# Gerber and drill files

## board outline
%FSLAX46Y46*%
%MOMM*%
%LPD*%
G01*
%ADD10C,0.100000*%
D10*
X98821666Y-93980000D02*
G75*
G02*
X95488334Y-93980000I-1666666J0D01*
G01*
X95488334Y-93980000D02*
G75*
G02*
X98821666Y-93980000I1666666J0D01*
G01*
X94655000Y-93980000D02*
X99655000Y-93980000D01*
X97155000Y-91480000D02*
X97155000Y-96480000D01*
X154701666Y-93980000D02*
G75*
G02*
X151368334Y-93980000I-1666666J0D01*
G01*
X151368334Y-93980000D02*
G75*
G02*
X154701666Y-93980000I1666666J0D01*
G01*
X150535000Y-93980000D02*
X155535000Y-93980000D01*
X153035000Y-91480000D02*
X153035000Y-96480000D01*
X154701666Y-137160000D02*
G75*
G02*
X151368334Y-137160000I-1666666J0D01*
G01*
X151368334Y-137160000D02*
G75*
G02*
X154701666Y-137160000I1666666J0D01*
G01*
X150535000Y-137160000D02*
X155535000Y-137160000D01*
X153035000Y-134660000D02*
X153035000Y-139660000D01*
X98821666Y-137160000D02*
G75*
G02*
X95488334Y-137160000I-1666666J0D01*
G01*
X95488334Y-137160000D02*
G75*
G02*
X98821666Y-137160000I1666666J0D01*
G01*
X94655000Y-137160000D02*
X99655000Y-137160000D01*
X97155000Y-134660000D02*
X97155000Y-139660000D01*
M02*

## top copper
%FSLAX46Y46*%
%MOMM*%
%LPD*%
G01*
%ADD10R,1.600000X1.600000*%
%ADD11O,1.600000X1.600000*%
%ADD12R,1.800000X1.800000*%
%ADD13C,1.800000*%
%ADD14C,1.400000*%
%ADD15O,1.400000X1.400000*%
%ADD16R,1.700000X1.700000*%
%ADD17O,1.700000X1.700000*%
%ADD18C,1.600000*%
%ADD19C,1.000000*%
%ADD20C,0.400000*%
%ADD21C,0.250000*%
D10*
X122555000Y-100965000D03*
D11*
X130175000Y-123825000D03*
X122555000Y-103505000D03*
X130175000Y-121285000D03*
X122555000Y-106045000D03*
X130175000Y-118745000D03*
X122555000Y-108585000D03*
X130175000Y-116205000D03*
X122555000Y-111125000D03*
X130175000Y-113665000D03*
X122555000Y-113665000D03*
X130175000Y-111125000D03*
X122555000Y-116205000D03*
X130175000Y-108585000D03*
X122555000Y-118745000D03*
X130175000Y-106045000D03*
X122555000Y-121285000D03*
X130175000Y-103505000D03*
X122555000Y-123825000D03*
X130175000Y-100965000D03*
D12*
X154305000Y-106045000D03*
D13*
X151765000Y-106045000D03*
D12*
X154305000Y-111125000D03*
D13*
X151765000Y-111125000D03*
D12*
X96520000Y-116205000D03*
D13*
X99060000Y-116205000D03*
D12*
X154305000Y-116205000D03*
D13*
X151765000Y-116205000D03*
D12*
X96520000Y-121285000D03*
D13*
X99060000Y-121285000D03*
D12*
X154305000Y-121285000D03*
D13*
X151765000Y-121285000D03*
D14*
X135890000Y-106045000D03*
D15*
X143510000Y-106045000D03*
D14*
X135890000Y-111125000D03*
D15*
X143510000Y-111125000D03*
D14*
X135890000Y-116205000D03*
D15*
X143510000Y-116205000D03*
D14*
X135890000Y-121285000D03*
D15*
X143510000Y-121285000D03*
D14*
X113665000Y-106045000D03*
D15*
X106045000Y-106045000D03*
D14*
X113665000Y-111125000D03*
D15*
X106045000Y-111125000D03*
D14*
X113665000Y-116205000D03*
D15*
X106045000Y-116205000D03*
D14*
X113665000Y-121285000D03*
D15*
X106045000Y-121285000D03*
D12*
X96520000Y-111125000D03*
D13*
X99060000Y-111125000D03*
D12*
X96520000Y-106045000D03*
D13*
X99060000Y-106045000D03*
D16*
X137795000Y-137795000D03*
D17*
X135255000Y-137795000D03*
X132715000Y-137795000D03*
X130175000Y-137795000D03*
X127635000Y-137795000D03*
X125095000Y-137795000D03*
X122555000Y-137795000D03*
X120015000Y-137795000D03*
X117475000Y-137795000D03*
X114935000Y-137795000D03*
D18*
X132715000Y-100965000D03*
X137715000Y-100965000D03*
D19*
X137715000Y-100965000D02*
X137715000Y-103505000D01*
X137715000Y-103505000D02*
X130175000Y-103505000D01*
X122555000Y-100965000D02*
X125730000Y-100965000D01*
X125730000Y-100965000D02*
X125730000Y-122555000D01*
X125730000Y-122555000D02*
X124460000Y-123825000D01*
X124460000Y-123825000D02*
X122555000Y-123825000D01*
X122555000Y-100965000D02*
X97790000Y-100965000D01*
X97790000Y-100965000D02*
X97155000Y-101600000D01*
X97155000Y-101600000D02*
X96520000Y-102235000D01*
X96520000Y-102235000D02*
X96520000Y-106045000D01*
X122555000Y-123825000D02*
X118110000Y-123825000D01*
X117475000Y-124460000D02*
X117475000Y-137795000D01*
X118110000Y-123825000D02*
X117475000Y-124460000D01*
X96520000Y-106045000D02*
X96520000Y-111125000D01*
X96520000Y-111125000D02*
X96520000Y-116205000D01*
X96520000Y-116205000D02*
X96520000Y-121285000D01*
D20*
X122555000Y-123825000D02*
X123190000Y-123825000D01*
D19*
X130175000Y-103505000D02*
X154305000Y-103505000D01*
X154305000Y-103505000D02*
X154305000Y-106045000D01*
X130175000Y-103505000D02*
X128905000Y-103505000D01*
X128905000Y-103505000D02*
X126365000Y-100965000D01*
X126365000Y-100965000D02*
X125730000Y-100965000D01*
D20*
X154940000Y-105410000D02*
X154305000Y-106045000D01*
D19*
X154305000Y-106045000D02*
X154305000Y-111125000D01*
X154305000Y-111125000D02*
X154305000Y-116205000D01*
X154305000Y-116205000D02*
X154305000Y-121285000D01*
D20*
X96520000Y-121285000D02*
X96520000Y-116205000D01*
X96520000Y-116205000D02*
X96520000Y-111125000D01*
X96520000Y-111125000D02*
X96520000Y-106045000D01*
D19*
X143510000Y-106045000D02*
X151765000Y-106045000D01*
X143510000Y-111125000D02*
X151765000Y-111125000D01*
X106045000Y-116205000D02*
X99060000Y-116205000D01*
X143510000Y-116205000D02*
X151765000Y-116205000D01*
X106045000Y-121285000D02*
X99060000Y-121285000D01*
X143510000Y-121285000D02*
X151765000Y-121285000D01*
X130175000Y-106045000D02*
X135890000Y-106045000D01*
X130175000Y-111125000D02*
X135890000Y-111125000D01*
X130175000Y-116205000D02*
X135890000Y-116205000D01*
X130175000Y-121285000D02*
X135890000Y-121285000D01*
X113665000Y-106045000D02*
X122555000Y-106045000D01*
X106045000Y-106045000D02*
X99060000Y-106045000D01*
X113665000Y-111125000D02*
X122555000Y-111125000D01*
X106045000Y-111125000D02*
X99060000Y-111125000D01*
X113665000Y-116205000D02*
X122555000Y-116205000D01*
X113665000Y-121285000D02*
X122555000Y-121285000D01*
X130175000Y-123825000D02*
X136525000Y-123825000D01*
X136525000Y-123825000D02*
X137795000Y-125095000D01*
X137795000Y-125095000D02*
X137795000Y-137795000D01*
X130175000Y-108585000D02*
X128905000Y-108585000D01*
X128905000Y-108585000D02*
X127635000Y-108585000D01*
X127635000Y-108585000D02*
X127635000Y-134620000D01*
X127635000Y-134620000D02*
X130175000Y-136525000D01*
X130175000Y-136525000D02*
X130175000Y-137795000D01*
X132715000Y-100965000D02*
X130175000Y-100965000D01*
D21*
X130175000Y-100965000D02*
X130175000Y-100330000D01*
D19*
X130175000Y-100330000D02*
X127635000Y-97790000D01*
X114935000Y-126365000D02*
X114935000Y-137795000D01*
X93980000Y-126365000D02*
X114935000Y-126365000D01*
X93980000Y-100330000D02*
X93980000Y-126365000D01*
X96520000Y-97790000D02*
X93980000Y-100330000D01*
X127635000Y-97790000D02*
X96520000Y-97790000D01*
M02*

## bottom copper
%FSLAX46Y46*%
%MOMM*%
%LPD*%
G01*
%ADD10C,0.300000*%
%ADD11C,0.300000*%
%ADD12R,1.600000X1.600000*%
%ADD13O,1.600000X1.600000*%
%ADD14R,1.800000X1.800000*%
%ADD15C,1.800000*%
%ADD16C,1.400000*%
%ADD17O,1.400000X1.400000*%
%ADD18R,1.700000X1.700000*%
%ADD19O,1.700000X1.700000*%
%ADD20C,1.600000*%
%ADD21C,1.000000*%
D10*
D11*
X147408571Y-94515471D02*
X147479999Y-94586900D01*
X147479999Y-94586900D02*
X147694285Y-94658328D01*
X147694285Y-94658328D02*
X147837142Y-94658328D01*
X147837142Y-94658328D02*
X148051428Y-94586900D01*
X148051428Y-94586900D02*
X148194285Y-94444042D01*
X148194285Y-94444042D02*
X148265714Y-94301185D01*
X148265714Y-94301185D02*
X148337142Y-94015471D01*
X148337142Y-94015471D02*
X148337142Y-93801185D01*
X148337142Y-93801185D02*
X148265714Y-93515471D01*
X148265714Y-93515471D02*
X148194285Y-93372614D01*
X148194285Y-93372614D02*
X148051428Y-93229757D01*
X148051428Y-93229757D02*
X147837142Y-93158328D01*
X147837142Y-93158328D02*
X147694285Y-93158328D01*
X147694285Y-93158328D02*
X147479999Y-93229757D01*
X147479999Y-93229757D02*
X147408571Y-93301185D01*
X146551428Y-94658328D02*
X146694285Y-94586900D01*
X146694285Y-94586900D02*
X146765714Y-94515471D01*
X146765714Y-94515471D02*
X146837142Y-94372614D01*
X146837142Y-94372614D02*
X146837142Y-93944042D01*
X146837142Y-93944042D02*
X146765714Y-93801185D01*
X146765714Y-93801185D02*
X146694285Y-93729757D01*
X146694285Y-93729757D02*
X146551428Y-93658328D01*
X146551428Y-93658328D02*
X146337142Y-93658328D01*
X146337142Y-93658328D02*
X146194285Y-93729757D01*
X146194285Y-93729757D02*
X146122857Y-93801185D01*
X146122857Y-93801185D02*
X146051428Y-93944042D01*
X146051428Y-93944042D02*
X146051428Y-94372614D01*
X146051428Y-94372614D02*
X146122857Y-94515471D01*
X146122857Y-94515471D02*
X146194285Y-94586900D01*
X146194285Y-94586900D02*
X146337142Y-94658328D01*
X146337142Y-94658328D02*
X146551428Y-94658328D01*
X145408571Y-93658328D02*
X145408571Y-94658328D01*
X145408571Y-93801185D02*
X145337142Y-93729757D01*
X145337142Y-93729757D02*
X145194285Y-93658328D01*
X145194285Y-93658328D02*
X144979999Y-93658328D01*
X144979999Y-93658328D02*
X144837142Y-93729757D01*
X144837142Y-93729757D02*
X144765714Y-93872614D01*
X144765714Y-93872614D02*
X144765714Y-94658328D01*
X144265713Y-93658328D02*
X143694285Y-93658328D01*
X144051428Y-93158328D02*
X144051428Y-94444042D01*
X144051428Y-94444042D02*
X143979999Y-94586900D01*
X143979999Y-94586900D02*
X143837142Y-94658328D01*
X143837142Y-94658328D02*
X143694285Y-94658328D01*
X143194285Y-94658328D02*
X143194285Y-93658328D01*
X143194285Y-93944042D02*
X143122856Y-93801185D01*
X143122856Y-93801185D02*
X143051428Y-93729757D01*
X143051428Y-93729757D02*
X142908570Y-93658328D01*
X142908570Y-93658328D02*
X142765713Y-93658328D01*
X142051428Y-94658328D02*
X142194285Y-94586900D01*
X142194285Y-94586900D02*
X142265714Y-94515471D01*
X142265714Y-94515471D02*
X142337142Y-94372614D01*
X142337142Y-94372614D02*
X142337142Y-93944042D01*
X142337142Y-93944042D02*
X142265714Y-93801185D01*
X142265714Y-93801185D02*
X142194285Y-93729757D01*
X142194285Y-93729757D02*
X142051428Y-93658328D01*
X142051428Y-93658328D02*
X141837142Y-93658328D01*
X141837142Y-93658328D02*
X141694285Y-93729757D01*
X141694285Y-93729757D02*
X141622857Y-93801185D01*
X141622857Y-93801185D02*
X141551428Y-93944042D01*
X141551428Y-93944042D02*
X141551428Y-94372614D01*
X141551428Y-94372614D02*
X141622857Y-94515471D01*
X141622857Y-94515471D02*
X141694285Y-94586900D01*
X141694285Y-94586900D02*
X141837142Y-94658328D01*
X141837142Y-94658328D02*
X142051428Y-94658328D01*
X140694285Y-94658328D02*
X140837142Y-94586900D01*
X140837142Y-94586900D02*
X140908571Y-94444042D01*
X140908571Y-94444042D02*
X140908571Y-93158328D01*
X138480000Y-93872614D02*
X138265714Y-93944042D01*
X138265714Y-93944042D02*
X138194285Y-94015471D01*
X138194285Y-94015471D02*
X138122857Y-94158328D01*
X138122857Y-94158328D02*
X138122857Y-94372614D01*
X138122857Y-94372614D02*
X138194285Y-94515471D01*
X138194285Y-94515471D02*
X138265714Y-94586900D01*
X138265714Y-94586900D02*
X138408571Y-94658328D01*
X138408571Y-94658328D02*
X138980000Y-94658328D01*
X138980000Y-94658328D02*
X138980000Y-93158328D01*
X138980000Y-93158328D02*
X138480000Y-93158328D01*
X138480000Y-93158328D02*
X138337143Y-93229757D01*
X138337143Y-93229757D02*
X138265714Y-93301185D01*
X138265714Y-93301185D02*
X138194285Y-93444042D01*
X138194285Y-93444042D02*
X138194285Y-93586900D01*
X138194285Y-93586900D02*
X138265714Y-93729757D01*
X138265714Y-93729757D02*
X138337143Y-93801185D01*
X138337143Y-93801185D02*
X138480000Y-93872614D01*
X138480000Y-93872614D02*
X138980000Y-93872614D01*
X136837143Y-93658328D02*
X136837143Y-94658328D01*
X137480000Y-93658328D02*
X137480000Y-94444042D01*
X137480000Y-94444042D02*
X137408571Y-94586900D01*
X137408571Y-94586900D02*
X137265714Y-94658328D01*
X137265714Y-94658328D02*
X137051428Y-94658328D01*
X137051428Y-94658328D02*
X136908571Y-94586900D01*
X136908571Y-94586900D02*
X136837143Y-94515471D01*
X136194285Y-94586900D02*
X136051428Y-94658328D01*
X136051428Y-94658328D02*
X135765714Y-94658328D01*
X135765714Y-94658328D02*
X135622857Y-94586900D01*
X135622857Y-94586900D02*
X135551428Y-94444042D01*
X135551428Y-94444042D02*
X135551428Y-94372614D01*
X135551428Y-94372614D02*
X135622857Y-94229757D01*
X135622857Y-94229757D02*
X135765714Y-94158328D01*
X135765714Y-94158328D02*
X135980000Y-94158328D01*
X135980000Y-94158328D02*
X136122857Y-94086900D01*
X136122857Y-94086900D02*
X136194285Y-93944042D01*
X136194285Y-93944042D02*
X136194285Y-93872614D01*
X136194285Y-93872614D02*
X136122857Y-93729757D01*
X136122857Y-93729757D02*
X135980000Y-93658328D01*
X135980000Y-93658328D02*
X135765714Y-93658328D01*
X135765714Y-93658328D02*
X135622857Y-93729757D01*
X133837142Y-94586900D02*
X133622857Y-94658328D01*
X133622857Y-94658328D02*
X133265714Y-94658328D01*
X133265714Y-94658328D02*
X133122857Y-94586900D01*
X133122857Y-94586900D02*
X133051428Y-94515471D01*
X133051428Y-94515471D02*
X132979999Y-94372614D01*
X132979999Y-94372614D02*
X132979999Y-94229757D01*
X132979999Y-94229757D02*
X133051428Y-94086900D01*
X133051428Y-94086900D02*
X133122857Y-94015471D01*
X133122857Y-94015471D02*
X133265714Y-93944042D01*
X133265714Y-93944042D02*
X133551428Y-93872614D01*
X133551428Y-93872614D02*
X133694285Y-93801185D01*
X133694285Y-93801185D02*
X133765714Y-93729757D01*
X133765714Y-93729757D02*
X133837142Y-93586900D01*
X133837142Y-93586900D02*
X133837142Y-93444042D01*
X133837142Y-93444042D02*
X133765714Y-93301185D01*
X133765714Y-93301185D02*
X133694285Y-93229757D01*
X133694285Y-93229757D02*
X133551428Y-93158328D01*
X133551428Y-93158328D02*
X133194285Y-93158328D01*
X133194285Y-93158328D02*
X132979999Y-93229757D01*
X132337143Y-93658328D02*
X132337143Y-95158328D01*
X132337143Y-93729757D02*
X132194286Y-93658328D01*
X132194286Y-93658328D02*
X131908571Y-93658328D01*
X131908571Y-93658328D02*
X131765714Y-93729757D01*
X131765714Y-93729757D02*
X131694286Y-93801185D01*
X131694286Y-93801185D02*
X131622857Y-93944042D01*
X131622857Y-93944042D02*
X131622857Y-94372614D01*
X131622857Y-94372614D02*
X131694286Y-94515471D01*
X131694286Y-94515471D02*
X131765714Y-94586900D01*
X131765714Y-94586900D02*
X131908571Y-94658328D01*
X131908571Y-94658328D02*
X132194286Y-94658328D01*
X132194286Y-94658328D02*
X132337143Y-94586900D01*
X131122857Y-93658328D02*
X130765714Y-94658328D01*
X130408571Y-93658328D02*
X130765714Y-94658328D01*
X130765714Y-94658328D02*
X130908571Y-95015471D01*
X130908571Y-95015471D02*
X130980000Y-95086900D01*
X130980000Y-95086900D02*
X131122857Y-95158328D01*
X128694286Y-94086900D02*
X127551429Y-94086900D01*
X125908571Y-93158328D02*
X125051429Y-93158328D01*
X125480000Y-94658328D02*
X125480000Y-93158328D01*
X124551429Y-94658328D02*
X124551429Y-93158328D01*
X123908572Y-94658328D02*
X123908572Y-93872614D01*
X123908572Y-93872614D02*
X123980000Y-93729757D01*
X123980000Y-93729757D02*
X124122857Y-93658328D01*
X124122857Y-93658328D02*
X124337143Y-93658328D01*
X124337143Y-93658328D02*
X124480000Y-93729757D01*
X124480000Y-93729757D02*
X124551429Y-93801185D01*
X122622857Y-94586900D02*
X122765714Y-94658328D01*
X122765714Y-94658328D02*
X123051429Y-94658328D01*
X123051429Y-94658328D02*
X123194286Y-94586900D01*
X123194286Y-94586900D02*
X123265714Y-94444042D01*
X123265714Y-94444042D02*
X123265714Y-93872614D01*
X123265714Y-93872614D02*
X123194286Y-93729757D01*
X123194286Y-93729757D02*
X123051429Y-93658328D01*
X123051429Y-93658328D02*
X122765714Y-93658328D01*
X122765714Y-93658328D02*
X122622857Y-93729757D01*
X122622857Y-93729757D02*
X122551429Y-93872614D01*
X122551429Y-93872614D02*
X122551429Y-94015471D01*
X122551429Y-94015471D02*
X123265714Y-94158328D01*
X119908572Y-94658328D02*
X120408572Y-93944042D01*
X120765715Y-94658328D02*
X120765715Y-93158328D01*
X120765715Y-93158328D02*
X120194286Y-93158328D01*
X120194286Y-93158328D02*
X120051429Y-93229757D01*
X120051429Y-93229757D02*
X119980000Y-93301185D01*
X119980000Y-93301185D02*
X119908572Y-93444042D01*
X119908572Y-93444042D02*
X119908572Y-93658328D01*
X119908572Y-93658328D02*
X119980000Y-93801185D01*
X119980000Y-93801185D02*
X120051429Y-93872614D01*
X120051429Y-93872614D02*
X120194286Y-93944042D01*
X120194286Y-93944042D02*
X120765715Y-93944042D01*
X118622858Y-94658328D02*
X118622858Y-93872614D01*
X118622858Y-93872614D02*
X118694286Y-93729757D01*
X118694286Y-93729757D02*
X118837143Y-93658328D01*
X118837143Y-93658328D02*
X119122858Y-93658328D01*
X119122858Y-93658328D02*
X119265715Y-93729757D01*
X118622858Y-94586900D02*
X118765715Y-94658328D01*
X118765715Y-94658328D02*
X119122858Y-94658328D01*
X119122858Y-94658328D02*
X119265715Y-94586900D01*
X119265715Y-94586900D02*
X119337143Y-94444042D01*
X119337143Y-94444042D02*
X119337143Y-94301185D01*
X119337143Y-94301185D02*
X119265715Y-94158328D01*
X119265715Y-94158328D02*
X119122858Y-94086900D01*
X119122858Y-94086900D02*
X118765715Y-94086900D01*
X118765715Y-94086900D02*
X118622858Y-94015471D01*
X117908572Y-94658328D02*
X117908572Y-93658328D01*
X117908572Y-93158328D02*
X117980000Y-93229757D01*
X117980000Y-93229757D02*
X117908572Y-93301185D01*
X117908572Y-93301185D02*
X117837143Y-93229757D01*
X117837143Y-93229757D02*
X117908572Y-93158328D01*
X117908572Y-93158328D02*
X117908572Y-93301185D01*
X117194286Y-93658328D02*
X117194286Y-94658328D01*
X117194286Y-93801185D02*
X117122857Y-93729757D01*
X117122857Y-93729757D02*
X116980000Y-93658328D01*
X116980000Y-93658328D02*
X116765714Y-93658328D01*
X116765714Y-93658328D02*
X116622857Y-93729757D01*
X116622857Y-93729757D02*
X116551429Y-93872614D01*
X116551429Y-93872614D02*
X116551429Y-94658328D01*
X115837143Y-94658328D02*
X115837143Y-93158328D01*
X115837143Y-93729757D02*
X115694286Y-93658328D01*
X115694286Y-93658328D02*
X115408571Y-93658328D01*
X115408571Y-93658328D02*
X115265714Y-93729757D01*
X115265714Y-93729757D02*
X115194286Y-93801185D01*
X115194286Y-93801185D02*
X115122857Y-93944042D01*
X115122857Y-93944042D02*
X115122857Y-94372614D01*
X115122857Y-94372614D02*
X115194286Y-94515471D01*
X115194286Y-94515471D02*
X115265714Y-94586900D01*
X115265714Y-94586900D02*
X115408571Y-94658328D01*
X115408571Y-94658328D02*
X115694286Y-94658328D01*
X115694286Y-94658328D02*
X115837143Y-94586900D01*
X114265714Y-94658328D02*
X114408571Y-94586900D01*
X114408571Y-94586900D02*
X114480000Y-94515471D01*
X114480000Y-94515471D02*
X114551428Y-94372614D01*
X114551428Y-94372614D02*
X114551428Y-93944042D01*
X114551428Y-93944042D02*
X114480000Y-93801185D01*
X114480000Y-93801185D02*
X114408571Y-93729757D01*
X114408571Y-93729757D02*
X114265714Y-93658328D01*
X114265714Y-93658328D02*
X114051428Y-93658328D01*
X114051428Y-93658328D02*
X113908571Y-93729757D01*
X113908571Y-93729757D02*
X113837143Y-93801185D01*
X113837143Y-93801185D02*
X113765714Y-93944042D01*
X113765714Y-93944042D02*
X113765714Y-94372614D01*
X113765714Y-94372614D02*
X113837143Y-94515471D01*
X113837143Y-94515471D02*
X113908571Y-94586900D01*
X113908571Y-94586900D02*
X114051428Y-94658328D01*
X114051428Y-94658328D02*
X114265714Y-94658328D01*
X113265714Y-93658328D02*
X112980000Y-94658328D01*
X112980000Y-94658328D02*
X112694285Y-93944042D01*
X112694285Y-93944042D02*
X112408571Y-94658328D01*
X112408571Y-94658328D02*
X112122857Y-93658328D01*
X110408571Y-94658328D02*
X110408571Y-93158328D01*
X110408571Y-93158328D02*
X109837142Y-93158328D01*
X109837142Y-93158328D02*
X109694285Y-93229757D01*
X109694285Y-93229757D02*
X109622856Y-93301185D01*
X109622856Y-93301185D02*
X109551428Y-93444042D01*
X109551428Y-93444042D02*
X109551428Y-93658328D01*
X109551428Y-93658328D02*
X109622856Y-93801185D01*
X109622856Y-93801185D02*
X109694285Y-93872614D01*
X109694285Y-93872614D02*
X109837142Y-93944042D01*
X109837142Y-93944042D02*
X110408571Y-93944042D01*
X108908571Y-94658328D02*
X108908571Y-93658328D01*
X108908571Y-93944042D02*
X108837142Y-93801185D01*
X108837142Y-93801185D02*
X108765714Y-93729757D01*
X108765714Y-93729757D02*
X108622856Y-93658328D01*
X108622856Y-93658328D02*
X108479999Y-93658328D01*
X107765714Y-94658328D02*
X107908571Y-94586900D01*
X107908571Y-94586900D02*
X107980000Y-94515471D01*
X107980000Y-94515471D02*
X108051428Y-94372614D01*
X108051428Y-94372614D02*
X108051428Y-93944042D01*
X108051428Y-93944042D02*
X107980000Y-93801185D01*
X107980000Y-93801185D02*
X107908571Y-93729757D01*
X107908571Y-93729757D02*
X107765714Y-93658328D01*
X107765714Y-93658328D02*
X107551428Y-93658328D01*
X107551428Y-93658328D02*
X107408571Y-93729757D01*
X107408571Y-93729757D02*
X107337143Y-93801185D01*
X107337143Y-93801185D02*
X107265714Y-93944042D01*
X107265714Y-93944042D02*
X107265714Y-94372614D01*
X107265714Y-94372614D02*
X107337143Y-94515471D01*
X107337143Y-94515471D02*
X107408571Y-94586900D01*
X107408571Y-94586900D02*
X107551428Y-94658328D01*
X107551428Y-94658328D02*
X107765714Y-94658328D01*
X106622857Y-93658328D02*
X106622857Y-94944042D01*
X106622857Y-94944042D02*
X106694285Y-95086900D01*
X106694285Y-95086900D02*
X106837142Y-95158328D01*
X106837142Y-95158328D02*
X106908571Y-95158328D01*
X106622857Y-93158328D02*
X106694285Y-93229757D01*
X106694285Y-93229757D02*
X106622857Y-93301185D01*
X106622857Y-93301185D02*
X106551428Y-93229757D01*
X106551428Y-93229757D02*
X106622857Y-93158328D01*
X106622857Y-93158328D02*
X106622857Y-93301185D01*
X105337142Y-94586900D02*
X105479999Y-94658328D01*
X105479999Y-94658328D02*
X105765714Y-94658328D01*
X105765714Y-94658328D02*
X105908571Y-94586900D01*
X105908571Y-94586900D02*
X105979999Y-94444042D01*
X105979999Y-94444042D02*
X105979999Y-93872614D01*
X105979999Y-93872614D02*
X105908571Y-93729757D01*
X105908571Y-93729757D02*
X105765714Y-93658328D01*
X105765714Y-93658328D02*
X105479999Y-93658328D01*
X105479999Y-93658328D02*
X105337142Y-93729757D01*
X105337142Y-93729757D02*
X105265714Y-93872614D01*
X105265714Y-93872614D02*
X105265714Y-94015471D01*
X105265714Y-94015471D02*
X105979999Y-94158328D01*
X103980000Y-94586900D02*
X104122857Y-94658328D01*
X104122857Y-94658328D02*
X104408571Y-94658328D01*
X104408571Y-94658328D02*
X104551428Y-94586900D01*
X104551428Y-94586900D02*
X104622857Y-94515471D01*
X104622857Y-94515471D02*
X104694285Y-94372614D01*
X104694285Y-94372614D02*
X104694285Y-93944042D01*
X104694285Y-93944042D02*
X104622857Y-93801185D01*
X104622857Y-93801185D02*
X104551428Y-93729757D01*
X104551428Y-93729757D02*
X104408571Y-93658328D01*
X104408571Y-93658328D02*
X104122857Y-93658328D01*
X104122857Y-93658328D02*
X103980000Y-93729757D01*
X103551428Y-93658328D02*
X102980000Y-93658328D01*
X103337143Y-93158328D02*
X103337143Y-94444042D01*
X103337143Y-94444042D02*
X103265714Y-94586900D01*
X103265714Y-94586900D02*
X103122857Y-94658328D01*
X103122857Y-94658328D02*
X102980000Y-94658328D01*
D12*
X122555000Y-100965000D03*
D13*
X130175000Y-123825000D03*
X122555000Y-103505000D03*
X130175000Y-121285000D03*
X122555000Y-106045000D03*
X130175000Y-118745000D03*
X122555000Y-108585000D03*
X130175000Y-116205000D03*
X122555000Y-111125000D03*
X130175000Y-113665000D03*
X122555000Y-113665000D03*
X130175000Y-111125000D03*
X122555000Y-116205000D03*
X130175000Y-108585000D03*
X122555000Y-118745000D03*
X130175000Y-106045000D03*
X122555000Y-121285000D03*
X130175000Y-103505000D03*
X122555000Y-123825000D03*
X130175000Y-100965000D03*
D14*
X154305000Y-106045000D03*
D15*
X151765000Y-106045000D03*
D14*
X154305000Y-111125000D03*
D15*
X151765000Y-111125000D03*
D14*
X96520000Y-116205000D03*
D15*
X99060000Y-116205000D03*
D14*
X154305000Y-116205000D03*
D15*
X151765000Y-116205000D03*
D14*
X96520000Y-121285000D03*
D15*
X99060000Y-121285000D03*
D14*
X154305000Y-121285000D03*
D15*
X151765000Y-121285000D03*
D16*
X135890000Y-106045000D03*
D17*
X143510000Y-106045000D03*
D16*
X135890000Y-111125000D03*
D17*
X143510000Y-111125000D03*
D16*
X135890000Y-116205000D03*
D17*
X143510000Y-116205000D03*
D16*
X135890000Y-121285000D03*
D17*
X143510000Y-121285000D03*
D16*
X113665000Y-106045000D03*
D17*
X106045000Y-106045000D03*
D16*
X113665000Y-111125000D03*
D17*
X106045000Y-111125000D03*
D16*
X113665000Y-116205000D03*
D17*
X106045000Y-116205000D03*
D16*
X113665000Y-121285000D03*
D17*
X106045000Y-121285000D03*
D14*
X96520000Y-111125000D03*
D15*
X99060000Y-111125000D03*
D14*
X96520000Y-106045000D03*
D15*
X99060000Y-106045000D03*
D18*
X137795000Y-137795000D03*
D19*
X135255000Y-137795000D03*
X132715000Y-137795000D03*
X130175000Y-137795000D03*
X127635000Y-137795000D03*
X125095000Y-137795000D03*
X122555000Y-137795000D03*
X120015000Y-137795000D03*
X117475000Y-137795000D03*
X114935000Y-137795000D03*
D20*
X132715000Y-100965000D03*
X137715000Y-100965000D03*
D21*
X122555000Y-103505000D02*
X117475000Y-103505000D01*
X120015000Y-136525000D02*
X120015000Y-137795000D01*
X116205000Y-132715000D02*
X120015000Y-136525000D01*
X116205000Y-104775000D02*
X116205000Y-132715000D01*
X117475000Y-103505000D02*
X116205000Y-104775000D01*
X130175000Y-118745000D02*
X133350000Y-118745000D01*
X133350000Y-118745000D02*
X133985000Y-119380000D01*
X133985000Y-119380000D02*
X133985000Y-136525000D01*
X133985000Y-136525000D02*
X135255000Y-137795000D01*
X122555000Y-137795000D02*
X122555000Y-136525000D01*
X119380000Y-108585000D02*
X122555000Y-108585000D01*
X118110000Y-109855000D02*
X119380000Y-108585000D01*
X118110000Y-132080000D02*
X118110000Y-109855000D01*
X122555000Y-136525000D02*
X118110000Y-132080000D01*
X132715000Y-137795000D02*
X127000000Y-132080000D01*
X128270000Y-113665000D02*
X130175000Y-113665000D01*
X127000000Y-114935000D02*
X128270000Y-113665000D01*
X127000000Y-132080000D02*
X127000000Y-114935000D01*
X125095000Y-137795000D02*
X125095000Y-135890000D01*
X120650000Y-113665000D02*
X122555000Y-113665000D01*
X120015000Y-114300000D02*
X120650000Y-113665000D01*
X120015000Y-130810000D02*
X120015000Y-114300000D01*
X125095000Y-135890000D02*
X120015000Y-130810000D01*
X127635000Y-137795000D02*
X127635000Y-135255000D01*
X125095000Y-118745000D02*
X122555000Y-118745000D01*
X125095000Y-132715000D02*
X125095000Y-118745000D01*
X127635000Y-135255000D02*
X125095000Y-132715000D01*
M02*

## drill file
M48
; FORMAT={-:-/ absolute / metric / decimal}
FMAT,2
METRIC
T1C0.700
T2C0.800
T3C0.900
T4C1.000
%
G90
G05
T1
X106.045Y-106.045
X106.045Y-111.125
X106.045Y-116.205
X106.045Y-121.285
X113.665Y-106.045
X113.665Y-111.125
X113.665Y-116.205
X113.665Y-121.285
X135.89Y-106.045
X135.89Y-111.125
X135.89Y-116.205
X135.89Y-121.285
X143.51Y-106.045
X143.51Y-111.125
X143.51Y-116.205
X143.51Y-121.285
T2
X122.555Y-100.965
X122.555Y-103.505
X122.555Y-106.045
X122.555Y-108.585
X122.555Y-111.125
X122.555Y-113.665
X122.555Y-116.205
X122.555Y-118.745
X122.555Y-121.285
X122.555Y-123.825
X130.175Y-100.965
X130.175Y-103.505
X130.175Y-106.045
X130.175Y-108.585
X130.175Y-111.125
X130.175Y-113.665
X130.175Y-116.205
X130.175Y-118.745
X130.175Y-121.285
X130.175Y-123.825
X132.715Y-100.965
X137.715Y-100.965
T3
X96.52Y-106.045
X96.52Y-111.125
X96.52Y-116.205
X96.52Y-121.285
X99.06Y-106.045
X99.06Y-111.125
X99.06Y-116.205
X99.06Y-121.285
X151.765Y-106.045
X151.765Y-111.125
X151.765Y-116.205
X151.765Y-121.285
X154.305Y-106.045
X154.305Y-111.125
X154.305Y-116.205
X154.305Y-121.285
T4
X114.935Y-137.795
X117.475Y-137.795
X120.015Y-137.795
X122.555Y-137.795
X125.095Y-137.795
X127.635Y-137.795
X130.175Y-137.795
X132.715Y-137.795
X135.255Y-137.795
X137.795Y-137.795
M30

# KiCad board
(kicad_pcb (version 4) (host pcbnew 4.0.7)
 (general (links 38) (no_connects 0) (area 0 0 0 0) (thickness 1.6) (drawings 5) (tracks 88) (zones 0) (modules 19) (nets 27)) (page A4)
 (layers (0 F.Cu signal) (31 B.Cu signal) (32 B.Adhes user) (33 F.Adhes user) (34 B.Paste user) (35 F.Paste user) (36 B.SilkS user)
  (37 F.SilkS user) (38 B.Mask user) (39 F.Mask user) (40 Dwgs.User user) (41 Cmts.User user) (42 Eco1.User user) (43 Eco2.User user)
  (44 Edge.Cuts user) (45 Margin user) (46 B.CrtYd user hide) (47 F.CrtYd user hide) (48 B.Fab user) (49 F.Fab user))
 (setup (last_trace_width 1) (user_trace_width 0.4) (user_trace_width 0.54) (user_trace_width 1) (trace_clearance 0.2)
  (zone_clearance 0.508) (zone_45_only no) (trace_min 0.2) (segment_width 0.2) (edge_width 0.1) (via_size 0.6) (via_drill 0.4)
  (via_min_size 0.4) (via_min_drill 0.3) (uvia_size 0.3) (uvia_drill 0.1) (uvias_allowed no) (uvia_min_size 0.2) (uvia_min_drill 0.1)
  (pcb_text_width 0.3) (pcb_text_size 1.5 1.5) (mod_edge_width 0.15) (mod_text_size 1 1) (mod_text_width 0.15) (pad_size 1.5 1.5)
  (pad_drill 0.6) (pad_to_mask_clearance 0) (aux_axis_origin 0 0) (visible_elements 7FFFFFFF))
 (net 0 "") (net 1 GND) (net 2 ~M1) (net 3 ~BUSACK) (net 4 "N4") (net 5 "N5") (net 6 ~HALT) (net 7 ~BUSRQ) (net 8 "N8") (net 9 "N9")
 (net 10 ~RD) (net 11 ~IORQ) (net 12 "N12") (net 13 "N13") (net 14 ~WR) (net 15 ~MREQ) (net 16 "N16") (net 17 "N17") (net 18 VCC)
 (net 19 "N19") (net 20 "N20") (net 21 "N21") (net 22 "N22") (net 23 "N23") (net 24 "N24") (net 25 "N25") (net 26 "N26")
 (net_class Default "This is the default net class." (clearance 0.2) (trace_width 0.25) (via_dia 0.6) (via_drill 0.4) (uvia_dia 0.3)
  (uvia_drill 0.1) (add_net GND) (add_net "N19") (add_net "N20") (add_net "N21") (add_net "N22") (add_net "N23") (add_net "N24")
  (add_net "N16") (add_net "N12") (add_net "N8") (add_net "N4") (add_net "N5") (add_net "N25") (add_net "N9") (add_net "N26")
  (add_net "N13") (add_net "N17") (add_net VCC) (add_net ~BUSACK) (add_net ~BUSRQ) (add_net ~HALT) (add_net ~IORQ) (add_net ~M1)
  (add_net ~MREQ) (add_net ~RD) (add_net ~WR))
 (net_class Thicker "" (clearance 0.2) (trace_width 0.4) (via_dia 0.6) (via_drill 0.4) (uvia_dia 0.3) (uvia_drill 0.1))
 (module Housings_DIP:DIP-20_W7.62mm (layer F.Cu) (at 122.555 100.965)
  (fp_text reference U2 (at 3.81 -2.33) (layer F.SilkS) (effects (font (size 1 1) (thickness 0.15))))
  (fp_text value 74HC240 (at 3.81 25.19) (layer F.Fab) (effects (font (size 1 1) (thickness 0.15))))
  (pad 1 thru_hole rect (at 0 0) (size 1.6 1.6) (drill 0.8) (layers *.Cu *.Mask) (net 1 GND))
  (pad 11 thru_hole oval (at 7.62 22.86) (size 1.6 1.6) (drill 0.8) (layers *.Cu *.Mask) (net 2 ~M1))
  (pad 2 thru_hole oval (at 0 2.54) (size 1.6 1.6) (drill 0.8) (layers *.Cu *.Mask) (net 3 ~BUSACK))
  (pad 12 thru_hole oval (at 7.62 20.32) (size 1.6 1.6) (drill 0.8) (layers *.Cu *.Mask) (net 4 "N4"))
  (pad 3 thru_hole oval (at 0 5.08) (size 1.6 1.6) (drill 0.8) (layers *.Cu *.Mask) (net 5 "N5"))
  (pad 13 thru_hole oval (at 7.62 17.78) (size 1.6 1.6) (drill 0.8) (layers *.Cu *.Mask) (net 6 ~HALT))
  (pad 4 thru_hole oval (at 0 7.62) (size 1.6 1.6) (drill 0.8) (layers *.Cu *.Mask) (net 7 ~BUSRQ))
  (pad 14 thru_hole oval (at 7.62 15.24) (size 1.6 1.6) (drill 0.8) (layers *.Cu *.Mask) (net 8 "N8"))
  (pad 5 thru_hole oval (at 0 10.16) (size 1.6 1.6) (drill 0.8) (layers *.Cu *.Mask) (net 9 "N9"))
  (pad 15 thru_hole oval (at 7.62 12.7) (size 1.6 1.6) (drill 0.8) (layers *.Cu *.Mask) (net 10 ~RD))
  (pad 6 thru_hole oval (at 0 12.7) (size 1.6 1.6) (drill 0.8) (layers *.Cu *.Mask) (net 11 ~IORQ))
  (pad 16 thru_hole oval (at 7.62 10.16) (size 1.6 1.6) (drill 0.8) (layers *.Cu *.Mask) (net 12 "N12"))
  (pad 7 thru_hole oval (at 0 15.24) (size 1.6 1.6) (drill 0.8) (layers *.Cu *.Mask) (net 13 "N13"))
  (pad 17 thru_hole oval (at 7.62 7.62) (size 1.6 1.6) (drill 0.8) (layers *.Cu *.Mask) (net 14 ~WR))
  (pad 8 thru_hole oval (at 0 17.78) (size 1.6 1.6) (drill 0.8) (layers *.Cu *.Mask) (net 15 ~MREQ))
  (pad 18 thru_hole oval (at 7.62 5.08) (size 1.6 1.6) (drill 0.8) (layers *.Cu *.Mask) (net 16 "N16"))
  (pad 9 thru_hole oval (at 0 20.32) (size 1.6 1.6) (drill 0.8) (layers *.Cu *.Mask) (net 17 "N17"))
  (pad 19 thru_hole oval (at 7.62 2.54) (size 1.6 1.6) (drill 0.8) (layers *.Cu *.Mask) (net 1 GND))
  (pad 10 thru_hole oval (at 0 22.86) (size 1.6 1.6) (drill 0.8) (layers *.Cu *.Mask) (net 1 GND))
  (pad 20 thru_hole oval (at 7.62 0) (size 1.6 1.6) (drill 0.8) (layers *.Cu *.Mask) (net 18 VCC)))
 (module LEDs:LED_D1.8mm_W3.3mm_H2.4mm (layer F.Cu) (at 154.305 106.045 180)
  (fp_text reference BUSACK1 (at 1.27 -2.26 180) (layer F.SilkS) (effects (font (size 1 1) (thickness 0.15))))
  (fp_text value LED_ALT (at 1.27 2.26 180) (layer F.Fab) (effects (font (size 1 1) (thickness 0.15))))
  (pad 1 thru_hole rect (at 0 0 180) (size 1.8 1.8) (drill 0.9) (layers *.Cu *.Mask) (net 1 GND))
  (pad 2 thru_hole circle (at 2.54 0 180) (size 1.8 1.8) (drill 0.9) (layers *.Cu *.Mask) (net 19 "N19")))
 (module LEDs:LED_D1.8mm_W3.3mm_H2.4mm (layer F.Cu) (at 154.305 111.125 180)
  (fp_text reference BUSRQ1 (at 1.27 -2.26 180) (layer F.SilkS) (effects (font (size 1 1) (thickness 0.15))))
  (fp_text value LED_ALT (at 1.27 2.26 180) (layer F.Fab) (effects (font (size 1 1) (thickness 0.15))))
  (pad 1 thru_hole rect (at 0 0 180) (size 1.8 1.8) (drill 0.9) (layers *.Cu *.Mask) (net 1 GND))
  (pad 2 thru_hole circle (at 2.54 0 180) (size 1.8 1.8) (drill 0.9) (layers *.Cu *.Mask) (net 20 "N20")))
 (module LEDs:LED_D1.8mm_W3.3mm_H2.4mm (layer F.Cu) (at 96.52 116.205)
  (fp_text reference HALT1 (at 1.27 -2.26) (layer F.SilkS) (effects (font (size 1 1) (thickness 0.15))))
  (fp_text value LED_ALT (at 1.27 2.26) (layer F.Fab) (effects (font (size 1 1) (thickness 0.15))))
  (pad 1 thru_hole rect (at 0 0) (size 1.8 1.8) (drill 0.9) (layers *.Cu *.Mask) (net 1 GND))
  (pad 2 thru_hole circle (at 2.54 0) (size 1.8 1.8) (drill 0.9) (layers *.Cu *.Mask) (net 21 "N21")))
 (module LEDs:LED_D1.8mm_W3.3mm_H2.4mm (layer F.Cu) (at 154.305 116.205 180)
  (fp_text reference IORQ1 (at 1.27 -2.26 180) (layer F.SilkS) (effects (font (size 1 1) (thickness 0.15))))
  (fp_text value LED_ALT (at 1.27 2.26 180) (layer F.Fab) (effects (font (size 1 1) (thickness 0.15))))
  (pad 1 thru_hole rect (at 0 0 180) (size 1.8 1.8) (drill 0.9) (layers *.Cu *.Mask) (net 1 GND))
  (pad 2 thru_hole circle (at 2.54 0 180) (size 1.8 1.8) (drill 0.9) (layers *.Cu *.Mask) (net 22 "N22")))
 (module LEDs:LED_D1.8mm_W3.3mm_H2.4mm (layer F.Cu) (at 96.52 121.285)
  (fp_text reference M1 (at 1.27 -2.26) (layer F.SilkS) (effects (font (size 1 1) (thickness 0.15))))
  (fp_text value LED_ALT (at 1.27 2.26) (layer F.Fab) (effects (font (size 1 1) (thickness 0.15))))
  (pad 1 thru_hole rect (at 0 0) (size 1.8 1.8) (drill 0.9) (layers *.Cu *.Mask) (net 1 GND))
  (pad 2 thru_hole circle (at 2.54 0) (size 1.8 1.8) (drill 0.9) (layers *.Cu *.Mask) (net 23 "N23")))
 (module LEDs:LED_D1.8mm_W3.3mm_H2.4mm (layer F.Cu) (at 154.305 121.285 180)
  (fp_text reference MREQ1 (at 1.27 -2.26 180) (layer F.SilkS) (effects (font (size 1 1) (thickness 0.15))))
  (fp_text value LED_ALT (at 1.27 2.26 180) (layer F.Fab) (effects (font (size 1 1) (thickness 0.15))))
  (pad 1 thru_hole rect (at 0 0 180) (size 1.8 1.8) (drill 0.9) (layers *.Cu *.Mask) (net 1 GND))
  (pad 2 thru_hole circle (at 2.54 0 180) (size 1.8 1.8) (drill 0.9) (layers *.Cu *.Mask) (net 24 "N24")))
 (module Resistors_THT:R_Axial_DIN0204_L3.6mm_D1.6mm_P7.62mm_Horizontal (layer F.Cu) (at 135.89 106.045)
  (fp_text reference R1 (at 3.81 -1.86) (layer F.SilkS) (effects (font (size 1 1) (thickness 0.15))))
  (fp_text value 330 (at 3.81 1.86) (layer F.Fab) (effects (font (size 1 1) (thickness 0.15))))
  (pad 1 thru_hole circle (at 0 0) (size 1.4 1.4) (drill 0.7) (layers *.Cu *.Mask) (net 16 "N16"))
  (pad 2 thru_hole oval (at 7.62 0) (size 1.4 1.4) (drill 0.7) (layers *.Cu *.Mask) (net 19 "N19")))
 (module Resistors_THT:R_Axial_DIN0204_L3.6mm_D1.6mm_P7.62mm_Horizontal (layer F.Cu) (at 135.89 111.125)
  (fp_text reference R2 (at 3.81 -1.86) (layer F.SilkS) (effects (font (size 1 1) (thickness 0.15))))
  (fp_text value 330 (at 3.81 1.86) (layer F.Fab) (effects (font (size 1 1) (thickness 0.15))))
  (pad 1 thru_hole circle (at 0 0) (size 1.4 1.4) (drill 0.7) (layers *.Cu *.Mask) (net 12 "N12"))
  (pad 2 thru_hole oval (at 7.62 0) (size 1.4 1.4) (drill 0.7) (layers *.Cu *.Mask) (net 20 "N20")))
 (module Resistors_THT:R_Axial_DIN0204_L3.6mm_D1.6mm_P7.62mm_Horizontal (layer F.Cu) (at 135.89 116.205)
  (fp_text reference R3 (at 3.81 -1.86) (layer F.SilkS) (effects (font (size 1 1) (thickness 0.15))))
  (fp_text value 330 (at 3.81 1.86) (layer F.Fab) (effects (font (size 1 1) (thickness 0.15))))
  (pad 1 thru_hole circle (at 0 0) (size 1.4 1.4) (drill 0.7) (layers *.Cu *.Mask) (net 8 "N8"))
  (pad 2 thru_hole oval (at 7.62 0) (size 1.4 1.4) (drill 0.7) (layers *.Cu *.Mask) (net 22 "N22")))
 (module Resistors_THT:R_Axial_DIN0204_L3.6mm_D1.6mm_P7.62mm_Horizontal (layer F.Cu) (at 135.89 121.285)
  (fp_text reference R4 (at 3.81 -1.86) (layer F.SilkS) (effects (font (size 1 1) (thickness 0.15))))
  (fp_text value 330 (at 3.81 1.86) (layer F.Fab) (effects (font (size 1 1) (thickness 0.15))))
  (pad 1 thru_hole circle (at 0 0) (size 1.4 1.4) (drill 0.7) (layers *.Cu *.Mask) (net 4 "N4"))
  (pad 2 thru_hole oval (at 7.62 0) (size 1.4 1.4) (drill 0.7) (layers *.Cu *.Mask) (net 24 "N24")))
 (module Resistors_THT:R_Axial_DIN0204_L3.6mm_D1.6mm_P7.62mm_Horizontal (layer F.Cu) (at 113.665 106.045 180)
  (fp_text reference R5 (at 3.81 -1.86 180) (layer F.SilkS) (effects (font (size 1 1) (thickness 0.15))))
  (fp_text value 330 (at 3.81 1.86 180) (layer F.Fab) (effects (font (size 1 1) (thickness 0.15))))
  (pad 1 thru_hole circle (at 0 0 180) (size 1.4 1.4) (drill 0.7) (layers *.Cu *.Mask) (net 5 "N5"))
  (pad 2 thru_hole oval (at 7.62 0 180) (size 1.4 1.4) (drill 0.7) (layers *.Cu *.Mask) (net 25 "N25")))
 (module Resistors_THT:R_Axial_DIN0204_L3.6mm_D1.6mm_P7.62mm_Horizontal (layer F.Cu) (at 113.665 111.125 180)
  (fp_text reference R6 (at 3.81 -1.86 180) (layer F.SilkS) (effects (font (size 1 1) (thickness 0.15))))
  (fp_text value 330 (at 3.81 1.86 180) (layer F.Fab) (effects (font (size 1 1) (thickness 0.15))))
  (pad 1 thru_hole circle (at 0 0 180) (size 1.4 1.4) (drill 0.7) (layers *.Cu *.Mask) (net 9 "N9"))
  (pad 2 thru_hole oval (at 7.62 0 180) (size 1.4 1.4) (drill 0.7) (layers *.Cu *.Mask) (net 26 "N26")))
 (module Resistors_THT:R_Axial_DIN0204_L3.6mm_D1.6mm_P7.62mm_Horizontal (layer F.Cu) (at 113.665 116.205 180)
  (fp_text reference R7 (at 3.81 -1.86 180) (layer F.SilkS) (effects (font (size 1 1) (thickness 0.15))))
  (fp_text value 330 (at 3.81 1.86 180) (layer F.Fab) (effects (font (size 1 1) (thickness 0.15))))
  (pad 1 thru_hole circle (at 0 0 180) (size 1.4 1.4) (drill 0.7) (layers *.Cu *.Mask) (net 13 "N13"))
  (pad 2 thru_hole oval (at 7.62 0 180) (size 1.4 1.4) (drill 0.7) (layers *.Cu *.Mask) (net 21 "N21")))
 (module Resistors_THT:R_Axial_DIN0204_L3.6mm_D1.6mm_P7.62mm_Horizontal (layer F.Cu) (at 113.665 121.285 180)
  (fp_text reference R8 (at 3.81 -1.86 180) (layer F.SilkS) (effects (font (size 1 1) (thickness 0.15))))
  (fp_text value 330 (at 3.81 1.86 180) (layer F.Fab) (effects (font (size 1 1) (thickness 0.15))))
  (pad 1 thru_hole circle (at 0 0 180) (size 1.4 1.4) (drill 0.7) (layers *.Cu *.Mask) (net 17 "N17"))
  (pad 2 thru_hole oval (at 7.62 0 180) (size 1.4 1.4) (drill 0.7) (layers *.Cu *.Mask) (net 23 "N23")))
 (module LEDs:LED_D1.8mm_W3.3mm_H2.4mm (layer F.Cu) (at 96.52 111.125)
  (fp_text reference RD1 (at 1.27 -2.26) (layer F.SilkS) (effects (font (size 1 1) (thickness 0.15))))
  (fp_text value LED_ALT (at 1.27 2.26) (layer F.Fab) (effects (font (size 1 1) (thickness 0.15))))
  (pad 1 thru_hole rect (at 0 0) (size 1.8 1.8) (drill 0.9) (layers *.Cu *.Mask) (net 1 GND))
  (pad 2 thru_hole circle (at 2.54 0) (size 1.8 1.8) (drill 0.9) (layers *.Cu *.Mask) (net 26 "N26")))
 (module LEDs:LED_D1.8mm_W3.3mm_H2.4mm (layer F.Cu) (at 96.52 106.045)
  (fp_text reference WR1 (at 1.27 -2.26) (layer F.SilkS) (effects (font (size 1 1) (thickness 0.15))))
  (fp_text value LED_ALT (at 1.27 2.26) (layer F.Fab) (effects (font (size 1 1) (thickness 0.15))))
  (pad 1 thru_hole rect (at 0 0) (size 1.8 1.8) (drill 0.9) (layers *.Cu *.Mask) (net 1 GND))
  (pad 2 thru_hole circle (at 2.54 0) (size 1.8 1.8) (drill 0.9) (layers *.Cu *.Mask) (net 25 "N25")))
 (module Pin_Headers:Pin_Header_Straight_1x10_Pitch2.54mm (layer F.Cu) (at 137.795 137.795 270)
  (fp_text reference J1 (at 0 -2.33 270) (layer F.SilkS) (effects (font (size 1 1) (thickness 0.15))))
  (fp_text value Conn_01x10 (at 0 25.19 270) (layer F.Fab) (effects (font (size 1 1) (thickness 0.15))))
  (pad 1 thru_hole rect (at 0 0 270) (size 1.7 1.7) (drill 1) (layers *.Cu *.Mask) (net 2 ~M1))
  (pad 2 thru_hole oval (at 0 2.54 270) (size 1.7 1.7) (drill 1) (layers *.Cu *.Mask) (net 6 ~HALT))
  (pad 3 thru_hole oval (at 0 5.08 270) (size 1.7 1.7) (drill 1) (layers *.Cu *.Mask) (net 10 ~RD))
  (pad 4 thru_hole oval (at 0 7.62 270) (size 1.7 1.7) (drill 1) (layers *.Cu *.Mask) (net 14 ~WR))
  (pad 5 thru_hole oval (at 0 10.16 270) (size 1.7 1.7) (drill 1) (layers *.Cu *.Mask) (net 15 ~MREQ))
  (pad 6 thru_hole oval (at 0 12.7 270) (size 1.7 1.7) (drill 1) (layers *.Cu *.Mask) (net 11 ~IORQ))
  (pad 7 thru_hole oval (at 0 15.24 270) (size 1.7 1.7) (drill 1) (layers *.Cu *.Mask) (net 7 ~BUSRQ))
  (pad 8 thru_hole oval (at 0 17.78 270) (size 1.7 1.7) (drill 1) (layers *.Cu *.Mask) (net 3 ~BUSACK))
  (pad 9 thru_hole oval (at 0 20.32 270) (size 1.7 1.7) (drill 1) (layers *.Cu *.Mask) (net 1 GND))
  (pad 10 thru_hole oval (at 0 22.86 270) (size 1.7 1.7) (drill 1) (layers *.Cu *.Mask) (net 18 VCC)))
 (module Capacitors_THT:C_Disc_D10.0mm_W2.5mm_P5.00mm (layer F.Cu) (at 132.715 100.965)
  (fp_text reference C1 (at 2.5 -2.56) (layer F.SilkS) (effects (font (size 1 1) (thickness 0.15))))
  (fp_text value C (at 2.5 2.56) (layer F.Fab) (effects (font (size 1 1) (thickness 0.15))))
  (pad 1 thru_hole circle (at 0 0) (size 1.6 1.6) (drill 0.8) (layers *.Cu *.Mask) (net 18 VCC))
  (pad 2 thru_hole circle (at 5 0) (size 1.6 1.6) (drill 0.8) (layers *.Cu *.Mask) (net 1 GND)))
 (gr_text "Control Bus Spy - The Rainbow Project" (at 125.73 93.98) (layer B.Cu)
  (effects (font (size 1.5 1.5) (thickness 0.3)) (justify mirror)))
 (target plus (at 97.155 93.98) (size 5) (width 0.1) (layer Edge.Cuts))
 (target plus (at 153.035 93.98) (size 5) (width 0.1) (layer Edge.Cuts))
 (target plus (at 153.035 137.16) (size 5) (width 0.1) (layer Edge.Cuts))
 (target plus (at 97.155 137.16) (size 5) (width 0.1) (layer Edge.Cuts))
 (segment (start 137.715 100.965) (end 137.715 103.505) (width 1) (layer F.Cu) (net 1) (status 400000))
 (segment (start 137.715 103.505) (end 130.175 103.505) (width 1) (layer F.Cu) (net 1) (status 800000))
 (segment (start 122.555 100.965) (end 125.73 100.965) (width 1) (layer F.Cu) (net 1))
 (segment (start 125.73 100.965) (end 125.73 122.555) (width 1) (layer F.Cu) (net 1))
 (segment (start 125.73 122.555) (end 124.46 123.825) (width 1) (layer F.Cu) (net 1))
 (segment (start 124.46 123.825) (end 122.555 123.825) (width 1) (layer F.Cu) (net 1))
 (segment (start 122.555 100.965) (end 97.79 100.965) (width 1) (layer F.Cu) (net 1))
 (segment (start 97.79 100.965) (end 97.155 101.6) (width 1) (layer F.Cu) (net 1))
 (segment (start 97.155 101.6) (end 96.52 102.235) (width 1) (layer F.Cu) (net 1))
 (segment (start 96.52 102.235) (end 96.52 106.045) (width 1) (layer F.Cu) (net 1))
 (segment (start 122.555 123.825) (end 118.11 123.825) (width 1) (layer F.Cu) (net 1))
 (segment (start 117.475 124.46) (end 117.475 137.795) (width 1) (layer F.Cu) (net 1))
 (segment (start 118.11 123.825) (end 117.475 124.46) (width 1) (layer F.Cu) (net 1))
 (segment (start 96.52 106.045) (end 96.52 111.125) (width 1) (layer F.Cu) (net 1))
 (segment (start 96.52 111.125) (end 96.52 116.205) (width 1) (layer F.Cu) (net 1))
 (segment (start 96.52 116.205) (end 96.52 121.285) (width 1) (layer F.Cu) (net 1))
 (segment (start 122.555 123.825) (end 123.19 123.825) (width 0.4) (layer F.Cu) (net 1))
 (segment (start 130.175 103.505) (end 154.305 103.505) (width 1) (layer F.Cu) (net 1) (status 10))
 (segment (start 154.305 103.505) (end 154.305 106.045) (width 1) (layer F.Cu) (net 1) (status 20))
 (segment (start 130.175 103.505) (end 128.905 103.505) (width 1) (layer F.Cu) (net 1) (status 10))
 (segment (start 128.905 103.505) (end 126.365 100.965) (width 1) (layer F.Cu) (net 1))
 (segment (start 126.365 100.965) (end 125.73 100.965) (width 1) (layer F.Cu) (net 1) (status 20))
 (segment (start 154.94 105.41) (end 154.305 106.045) (width 0.4) (layer F.Cu) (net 1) (status 30))
 (segment (start 154.305 106.045) (end 154.305 111.125) (width 1) (layer F.Cu) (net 1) (status 30))
 (segment (start 154.305 111.125) (end 154.305 116.205) (width 1) (layer F.Cu) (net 1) (status 30))
 (segment (start 154.305 116.205) (end 154.305 121.285) (width 1) (layer F.Cu) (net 1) (status 30))
 (segment (start 96.52 121.285) (end 96.52 116.205) (width 0.4) (layer F.Cu) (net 1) (status 30))
 (segment (start 96.52 116.205) (end 96.52 111.125) (width 0.4) (layer F.Cu) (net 1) (status 30))
 (segment (start 96.52 111.125) (end 96.52 106.045) (width 0.4) (layer F.Cu) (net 1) (status 30))
 (segment (start 143.51 106.045) (end 151.765 106.045) (width 1) (layer F.Cu) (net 19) (status 30))
 (segment (start 143.51 111.125) (end 151.765 111.125) (width 1) (layer F.Cu) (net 20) (status 30))
 (segment (start 106.045 116.205) (end 99.06 116.205) (width 1) (layer F.Cu) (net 21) (status 30))
 (segment (start 143.51 116.205) (end 151.765 116.205) (width 1) (layer F.Cu) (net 22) (status 30))
 (segment (start 106.045 121.285) (end 99.06 121.285) (width 1) (layer F.Cu) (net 23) (status 30))
 (segment (start 143.51 121.285) (end 151.765 121.285) (width 1) (layer F.Cu) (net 24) (status 30))
 (segment (start 130.175 106.045) (end 135.89 106.045) (width 1) (layer F.Cu) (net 16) (status 30))
 (segment (start 130.175 111.125) (end 135.89 111.125) (width 1) (layer F.Cu) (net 12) (status 30))
 (segment (start 130.175 116.205) (end 135.89 116.205) (width 1) (layer F.Cu) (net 8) (status 30))
 (segment (start 130.175 121.285) (end 135.89 121.285) (width 1) (layer F.Cu) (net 4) (status 30))
 (segment (start 113.665 106.045) (end 122.555 106.045) (width 1) (layer F.Cu) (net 5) (status 30))
 (segment (start 106.045 106.045) (end 99.06 106.045) (width 1) (layer F.Cu) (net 25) (status 30))
 (segment (start 113.665 111.125) (end 122.555 111.125) (width 1) (layer F.Cu) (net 9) (status 30))
 (segment (start 106.045 111.125) (end 99.06 111.125) (width 1) (layer F.Cu) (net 26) (status 30))
 (segment (start 113.665 116.205) (end 122.555 116.205) (width 1) (layer F.Cu) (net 13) (status 30))
 (segment (start 113.665 121.285) (end 122.555 121.285) (width 1) (layer F.Cu) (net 17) (status 30))
 (segment (start 130.175 123.825) (end 136.525 123.825) (width 1) (layer F.Cu) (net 2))
 (segment (start 136.525 123.825) (end 137.795 125.095) (width 1) (layer F.Cu) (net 2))
 (segment (start 137.795 125.095) (end 137.795 137.795) (width 1) (layer F.Cu) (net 2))
 (segment (start 122.555 103.505) (end 117.475 103.505) (width 1) (layer B.Cu) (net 3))
 (segment (start 120.015 136.525) (end 120.015 137.795) (width 1) (layer B.Cu) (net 3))
 (segment (start 116.205 132.715) (end 120.015 136.525) (width 1) (layer B.Cu) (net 3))
 (segment (start 116.205 104.775) (end 116.205 132.715) (width 1) (layer B.Cu) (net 3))
 (segment (start 117.475 103.505) (end 116.205 104.775) (width 1) (layer B.Cu) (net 3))
 (segment (start 130.175 118.745) (end 133.35 118.745) (width 1) (layer B.Cu) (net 6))
 (segment (start 133.35 118.745) (end 133.985 119.38) (width 1) (layer B.Cu) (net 6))
 (segment (start 133.985 119.38) (end 133.985 136.525) (width 1) (layer B.Cu) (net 6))
 (segment (start 133.985 136.525) (end 135.255 137.795) (width 1) (layer B.Cu) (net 6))
 (segment (start 122.555 137.795) (end 122.555 136.525) (width 1) (layer B.Cu) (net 7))
 (segment (start 119.38 108.585) (end 122.555 108.585) (width 1) (layer B.Cu) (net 7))
 (segment (start 118.11 109.855) (end 119.38 108.585) (width 1) (layer B.Cu) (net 7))
 (segment (start 118.11 132.08) (end 118.11 109.855) (width 1) (layer B.Cu) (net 7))
 (segment (start 122.555 136.525) (end 118.11 132.08) (width 1) (layer B.Cu) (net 7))
 (segment (start 132.715 137.795) (end 127 132.08) (width 1) (layer B.Cu) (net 10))
 (segment (start 128.27 113.665) (end 130.175 113.665) (width 1) (layer B.Cu) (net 10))
 (segment (start 127 114.935) (end 128.27 113.665) (width 1) (layer B.Cu) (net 10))
 (segment (start 127 132.08) (end 127 114.935) (width 1) (layer B.Cu) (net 10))
 (segment (start 125.095 137.795) (end 125.095 135.89) (width 1) (layer B.Cu) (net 11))
 (segment (start 120.65 113.665) (end 122.555 113.665) (width 1) (layer B.Cu) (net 11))
 (segment (start 120.015 114.3) (end 120.65 113.665) (width 1) (layer B.Cu) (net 11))
 (segment (start 120.015 130.81) (end 120.015 114.3) (width 1) (layer B.Cu) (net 11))
 (segment (start 125.095 135.89) (end 120.015 130.81) (width 1) (layer B.Cu) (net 11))
 (segment (start 130.175 108.585) (end 128.905 108.585) (width 1) (layer F.Cu) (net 14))
 (segment (start 128.905 108.585) (end 127.635 108.585) (width 1) (layer F.Cu) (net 14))
 (segment (start 127.635 108.585) (end 127.635 134.62) (width 1) (layer F.Cu) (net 14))
 (segment (start 127.635 134.62) (end 130.175 136.525) (width 1) (layer F.Cu) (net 14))
 (segment (start 130.175 136.525) (end 130.175 137.795) (width 1) (layer F.Cu) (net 14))
 (segment (start 127.635 137.795) (end 127.635 135.255) (width 1) (layer B.Cu) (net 15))
 (segment (start 125.095 118.745) (end 122.555 118.745) (width 1) (layer B.Cu) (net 15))
 (segment (start 125.095 132.715) (end 125.095 118.745) (width 1) (layer B.Cu) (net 15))
 (segment (start 127.635 135.255) (end 125.095 132.715) (width 1) (layer B.Cu) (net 15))
 (segment (start 132.715 100.965) (end 130.175 100.965) (width 1) (layer F.Cu) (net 18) (status C00000))
 (segment (start 130.175 100.965) (end 130.175 100.33) (width 0.25) (layer F.Cu) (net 18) (status 30))
 (segment (start 130.175 100.33) (end 127.635 97.79) (width 1) (layer F.Cu) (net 18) (status 10))
 (segment (start 114.935 126.365) (end 114.935 137.795) (width 1) (layer F.Cu) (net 18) (status 20))
 (segment (start 93.98 126.365) (end 114.935 126.365) (width 1) (layer F.Cu) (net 18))
 (segment (start 93.98 100.33) (end 93.98 126.365) (width 1) (layer F.Cu) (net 18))
 (segment (start 96.52 97.79) (end 93.98 100.33) (width 1) (layer F.Cu) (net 18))
 (segment (start 127.635 97.79) (end 96.52 97.79) (width 1) (layer F.Cu) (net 18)))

